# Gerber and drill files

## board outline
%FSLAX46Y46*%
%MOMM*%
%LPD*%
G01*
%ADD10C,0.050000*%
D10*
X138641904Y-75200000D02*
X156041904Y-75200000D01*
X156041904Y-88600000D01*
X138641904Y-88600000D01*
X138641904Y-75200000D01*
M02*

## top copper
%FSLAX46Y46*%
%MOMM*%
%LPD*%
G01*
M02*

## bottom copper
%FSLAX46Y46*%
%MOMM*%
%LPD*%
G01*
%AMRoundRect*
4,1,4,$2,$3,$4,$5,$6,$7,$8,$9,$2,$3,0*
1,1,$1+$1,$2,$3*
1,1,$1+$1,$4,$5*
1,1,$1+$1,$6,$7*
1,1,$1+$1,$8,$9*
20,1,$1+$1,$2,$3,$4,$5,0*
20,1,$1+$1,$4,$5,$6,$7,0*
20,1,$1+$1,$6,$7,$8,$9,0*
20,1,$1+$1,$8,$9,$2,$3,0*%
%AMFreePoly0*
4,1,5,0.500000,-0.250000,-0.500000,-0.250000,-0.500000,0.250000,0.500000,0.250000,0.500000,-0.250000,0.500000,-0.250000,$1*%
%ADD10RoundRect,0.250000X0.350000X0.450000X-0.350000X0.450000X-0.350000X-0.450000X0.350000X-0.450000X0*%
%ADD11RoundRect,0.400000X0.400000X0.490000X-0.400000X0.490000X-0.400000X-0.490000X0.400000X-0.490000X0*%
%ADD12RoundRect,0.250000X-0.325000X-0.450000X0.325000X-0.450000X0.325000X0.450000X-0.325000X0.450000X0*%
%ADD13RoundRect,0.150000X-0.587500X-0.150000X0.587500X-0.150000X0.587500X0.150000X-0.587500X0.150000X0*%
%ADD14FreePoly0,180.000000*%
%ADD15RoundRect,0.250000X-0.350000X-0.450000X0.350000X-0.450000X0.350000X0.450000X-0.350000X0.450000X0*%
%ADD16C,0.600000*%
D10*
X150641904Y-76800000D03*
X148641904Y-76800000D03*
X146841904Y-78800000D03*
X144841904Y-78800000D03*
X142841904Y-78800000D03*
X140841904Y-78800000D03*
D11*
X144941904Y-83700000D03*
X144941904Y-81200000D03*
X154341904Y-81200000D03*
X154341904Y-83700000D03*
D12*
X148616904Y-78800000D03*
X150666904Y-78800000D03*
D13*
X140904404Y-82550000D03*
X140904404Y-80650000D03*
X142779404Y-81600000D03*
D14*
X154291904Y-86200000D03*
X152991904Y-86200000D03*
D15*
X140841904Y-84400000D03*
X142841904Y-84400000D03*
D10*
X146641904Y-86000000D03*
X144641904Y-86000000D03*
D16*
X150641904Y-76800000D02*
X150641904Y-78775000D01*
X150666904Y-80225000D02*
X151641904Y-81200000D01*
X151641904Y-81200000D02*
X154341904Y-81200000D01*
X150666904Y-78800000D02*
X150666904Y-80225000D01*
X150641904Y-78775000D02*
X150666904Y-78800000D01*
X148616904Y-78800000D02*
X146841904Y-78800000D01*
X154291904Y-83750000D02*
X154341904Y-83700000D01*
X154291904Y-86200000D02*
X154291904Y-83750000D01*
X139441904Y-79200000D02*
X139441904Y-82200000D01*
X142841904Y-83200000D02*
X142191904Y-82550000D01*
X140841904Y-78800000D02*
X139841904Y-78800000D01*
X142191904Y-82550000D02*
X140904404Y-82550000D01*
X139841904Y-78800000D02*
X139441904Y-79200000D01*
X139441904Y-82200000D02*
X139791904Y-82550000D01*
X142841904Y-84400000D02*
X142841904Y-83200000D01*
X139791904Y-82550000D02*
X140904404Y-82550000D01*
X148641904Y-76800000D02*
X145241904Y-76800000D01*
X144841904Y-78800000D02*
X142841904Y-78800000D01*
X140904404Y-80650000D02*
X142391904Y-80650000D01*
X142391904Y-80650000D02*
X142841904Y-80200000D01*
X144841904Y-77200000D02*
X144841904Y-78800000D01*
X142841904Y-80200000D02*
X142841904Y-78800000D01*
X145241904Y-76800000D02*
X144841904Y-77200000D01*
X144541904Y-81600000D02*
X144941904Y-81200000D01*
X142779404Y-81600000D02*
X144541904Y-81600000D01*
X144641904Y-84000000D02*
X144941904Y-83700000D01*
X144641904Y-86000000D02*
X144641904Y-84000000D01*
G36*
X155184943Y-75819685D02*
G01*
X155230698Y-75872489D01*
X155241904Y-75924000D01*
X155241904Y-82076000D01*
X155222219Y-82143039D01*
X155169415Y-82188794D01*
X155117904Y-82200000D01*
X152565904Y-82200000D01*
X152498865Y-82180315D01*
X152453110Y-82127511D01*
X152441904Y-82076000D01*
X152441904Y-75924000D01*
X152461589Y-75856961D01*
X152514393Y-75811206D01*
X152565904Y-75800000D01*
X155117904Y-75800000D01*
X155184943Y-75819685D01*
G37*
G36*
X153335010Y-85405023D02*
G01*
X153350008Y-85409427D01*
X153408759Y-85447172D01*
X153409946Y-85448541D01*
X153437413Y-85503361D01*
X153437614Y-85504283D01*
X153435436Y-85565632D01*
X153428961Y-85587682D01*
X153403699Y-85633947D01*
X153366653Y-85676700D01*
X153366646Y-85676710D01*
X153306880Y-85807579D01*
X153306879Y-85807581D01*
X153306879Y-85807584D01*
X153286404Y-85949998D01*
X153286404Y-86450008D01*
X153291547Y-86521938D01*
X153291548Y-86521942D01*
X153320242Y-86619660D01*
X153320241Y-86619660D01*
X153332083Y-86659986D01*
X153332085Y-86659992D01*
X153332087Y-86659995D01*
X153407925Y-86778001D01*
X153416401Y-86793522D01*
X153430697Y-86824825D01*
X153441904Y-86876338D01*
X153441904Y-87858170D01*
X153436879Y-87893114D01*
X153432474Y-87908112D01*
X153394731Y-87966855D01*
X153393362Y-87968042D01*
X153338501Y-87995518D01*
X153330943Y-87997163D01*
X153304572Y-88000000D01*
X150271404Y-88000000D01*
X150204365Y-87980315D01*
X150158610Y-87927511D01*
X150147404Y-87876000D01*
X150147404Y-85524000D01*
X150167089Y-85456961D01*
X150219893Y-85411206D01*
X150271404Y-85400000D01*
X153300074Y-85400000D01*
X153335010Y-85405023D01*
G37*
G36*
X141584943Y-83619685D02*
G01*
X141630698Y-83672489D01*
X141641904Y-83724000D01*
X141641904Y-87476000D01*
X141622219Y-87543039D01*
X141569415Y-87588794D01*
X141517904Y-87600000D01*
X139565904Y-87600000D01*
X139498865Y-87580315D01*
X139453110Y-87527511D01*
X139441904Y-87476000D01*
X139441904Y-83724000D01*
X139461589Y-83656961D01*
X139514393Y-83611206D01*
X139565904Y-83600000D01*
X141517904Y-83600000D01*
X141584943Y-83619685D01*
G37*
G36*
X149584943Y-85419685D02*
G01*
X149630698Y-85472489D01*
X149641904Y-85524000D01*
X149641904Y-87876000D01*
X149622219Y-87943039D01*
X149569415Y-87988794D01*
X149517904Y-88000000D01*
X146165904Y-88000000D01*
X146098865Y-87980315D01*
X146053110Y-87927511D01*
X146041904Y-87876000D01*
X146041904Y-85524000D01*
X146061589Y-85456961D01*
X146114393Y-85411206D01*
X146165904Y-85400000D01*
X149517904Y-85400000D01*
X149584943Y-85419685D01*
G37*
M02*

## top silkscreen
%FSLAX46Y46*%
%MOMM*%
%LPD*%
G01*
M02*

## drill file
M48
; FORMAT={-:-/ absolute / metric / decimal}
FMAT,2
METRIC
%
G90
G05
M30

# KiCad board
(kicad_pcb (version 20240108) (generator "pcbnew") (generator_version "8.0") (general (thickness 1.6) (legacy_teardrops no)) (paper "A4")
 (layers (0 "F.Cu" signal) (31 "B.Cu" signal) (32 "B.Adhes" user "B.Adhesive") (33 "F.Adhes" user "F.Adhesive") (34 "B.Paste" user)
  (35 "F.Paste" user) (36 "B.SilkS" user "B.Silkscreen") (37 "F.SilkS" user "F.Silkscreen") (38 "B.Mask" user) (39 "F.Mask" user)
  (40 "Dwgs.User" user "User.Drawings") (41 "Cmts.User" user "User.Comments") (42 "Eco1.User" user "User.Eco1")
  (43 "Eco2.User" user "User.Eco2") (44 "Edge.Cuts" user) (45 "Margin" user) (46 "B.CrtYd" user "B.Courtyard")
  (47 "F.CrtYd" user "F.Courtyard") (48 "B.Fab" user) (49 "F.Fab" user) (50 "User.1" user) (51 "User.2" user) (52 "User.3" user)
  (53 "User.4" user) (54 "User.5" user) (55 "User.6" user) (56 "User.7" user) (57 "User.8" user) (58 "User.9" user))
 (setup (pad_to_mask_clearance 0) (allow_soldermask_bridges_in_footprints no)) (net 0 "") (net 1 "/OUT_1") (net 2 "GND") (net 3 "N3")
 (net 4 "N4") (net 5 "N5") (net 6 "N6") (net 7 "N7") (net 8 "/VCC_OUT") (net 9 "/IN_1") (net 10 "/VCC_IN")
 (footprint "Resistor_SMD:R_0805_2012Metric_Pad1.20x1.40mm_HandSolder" (layer "B.Cu") (at 149.641904 76.8 180)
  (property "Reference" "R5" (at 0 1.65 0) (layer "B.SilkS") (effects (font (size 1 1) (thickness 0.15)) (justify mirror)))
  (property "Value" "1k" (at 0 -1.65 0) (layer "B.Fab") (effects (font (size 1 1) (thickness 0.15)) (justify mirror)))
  (pad "1" smd roundrect (at -1 0 180) (size 1.2 1.4) (layers "B.Cu" "B.Paste" "B.Mask") (roundrect_rratio 0.208333) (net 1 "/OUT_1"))
  (pad "2" smd roundrect (at 1 0 180) (size 1.2 1.4) (layers "B.Cu" "B.Paste" "B.Mask") (roundrect_rratio 0.208333) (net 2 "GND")))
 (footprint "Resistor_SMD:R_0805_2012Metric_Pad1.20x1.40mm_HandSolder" (layer "B.Cu") (at 145.841904 78.8 180)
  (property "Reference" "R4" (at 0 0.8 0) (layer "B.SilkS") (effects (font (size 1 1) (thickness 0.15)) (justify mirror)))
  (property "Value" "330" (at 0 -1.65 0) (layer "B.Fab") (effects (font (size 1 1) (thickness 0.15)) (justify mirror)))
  (pad "1" smd roundrect (at -1 0 180) (size 1.2 1.4) (layers "B.Cu" "B.Paste" "B.Mask") (roundrect_rratio 0.208333) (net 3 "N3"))
  (pad "2" smd roundrect (at 1 0 180) (size 1.2 1.4) (layers "B.Cu" "B.Paste" "B.Mask") (roundrect_rratio 0.208333) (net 2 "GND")))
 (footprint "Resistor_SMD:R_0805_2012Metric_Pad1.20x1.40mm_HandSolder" (layer "B.Cu") (at 141.841904 78.8 180)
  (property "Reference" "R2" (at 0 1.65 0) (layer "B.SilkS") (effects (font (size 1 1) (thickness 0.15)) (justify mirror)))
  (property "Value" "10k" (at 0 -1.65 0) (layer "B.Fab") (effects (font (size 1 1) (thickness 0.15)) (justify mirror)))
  (pad "1" smd roundrect (at -1 0 180) (size 1.2 1.4) (layers "B.Cu" "B.Paste" "B.Mask") (roundrect_rratio 0.208333) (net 2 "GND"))
  (pad "2" smd roundrect (at 1 0 180) (size 1.2 1.4) (layers "B.Cu" "B.Paste" "B.Mask") (roundrect_rratio 0.208333) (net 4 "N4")))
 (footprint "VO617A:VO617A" (layer "B.Cu") (at 149.641904 82.4 180)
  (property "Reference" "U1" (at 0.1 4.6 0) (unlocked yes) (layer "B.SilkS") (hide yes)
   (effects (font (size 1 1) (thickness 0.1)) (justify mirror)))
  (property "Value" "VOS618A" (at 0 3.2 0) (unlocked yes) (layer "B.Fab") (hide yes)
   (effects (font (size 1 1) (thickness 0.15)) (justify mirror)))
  (pad "1" smd roundrect (at 4.7 -1.3 180) (size 1.6 1.78) (layers "B.Cu" "B.Paste" "B.Mask") (roundrect_rratio 0.25) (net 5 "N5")
   (thermal_bridge_angle 45))
  (pad "2" smd roundrect (at 4.7 1.2 180) (size 1.6 1.78) (layers "B.Cu" "B.Paste" "B.Mask") (roundrect_rratio 0.25) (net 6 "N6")
   (thermal_bridge_angle 45))
  (pad "3" smd roundrect (at -4.7 1.2 180) (size 1.6 1.78) (layers "B.Cu" "B.Paste" "B.Mask") (roundrect_rratio 0.25) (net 1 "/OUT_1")
   (thermal_bridge_angle 45))
  (pad "4" smd roundrect (at -4.7 -1.3 180) (size 1.6 1.78) (layers "B.Cu" "B.Paste" "B.Mask") (roundrect_rratio 0.25) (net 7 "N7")
   (thermal_bridge_angle 45)))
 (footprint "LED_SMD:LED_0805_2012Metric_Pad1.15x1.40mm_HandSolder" (layer "B.Cu") (at 149.641904 78.8)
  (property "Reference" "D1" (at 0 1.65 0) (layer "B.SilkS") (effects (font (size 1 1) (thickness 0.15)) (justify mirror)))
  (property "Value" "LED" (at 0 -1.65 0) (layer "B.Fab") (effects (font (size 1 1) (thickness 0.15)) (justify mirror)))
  (pad "1" smd roundrect (at -1.025 0) (size 1.15 1.4) (layers "B.Cu" "B.Paste" "B.Mask") (roundrect_rratio 0.217391) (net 3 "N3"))
  (pad "2" smd roundrect (at 1.025 0) (size 1.15 1.4) (layers "B.Cu" "B.Paste" "B.Mask") (roundrect_rratio 0.217391) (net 1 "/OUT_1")))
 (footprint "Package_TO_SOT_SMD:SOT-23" (layer "B.Cu") (at 141.841904 81.6)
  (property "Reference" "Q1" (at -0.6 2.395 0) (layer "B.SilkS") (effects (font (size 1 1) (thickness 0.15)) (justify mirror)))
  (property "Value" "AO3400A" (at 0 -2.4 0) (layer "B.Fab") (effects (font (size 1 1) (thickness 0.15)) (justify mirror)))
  (pad "1" smd roundrect (at -0.9375 0.95) (size 1.475 0.6) (layers "B.Cu" "B.Paste" "B.Mask") (roundrect_rratio 0.25) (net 4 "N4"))
  (pad "2" smd roundrect (at -0.9375 -0.95) (size 1.475 0.6) (layers "B.Cu" "B.Paste" "B.Mask") (roundrect_rratio 0.25) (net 2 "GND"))
  (pad "3" smd roundrect (at 0.9375 0) (size 1.475 0.6) (layers "B.Cu" "B.Paste" "B.Mask") (roundrect_rratio 0.25) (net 6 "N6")))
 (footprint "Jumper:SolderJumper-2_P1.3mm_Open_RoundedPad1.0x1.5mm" (layer "B.Cu") (at 153.641904 86.2 180)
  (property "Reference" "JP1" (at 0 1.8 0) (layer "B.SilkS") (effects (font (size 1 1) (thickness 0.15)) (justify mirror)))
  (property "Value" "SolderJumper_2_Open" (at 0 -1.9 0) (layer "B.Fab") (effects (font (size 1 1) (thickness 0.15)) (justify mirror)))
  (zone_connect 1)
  (pad "1" smd custom (at -0.65 0 180) (size 1 0.5) (layers "B.Cu" "B.Mask") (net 7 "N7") (zone_connect 2) (thermal_bridge_angle 45)
   (options (clearance outline) (anchor rect)) (primitives))
  (pad "2" smd custom (at 0.65 0 180) (size 1 0.5) (layers "B.Cu" "B.Mask") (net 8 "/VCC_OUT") (zone_connect 2) (thermal_bridge_angle 45)
   (options (clearance outline) (anchor rect)) (primitives)))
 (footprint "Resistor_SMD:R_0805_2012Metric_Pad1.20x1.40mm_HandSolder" (layer "B.Cu") (at 141.841904 84.4)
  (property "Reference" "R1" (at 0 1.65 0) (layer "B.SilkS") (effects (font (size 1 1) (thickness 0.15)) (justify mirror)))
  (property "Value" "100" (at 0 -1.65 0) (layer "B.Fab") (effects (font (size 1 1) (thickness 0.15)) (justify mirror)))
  (pad "1" smd roundrect (at -1 0) (size 1.2 1.4) (layers "B.Cu" "B.Paste" "B.Mask") (roundrect_rratio 0.208333) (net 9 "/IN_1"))
  (pad "2" smd roundrect (at 1 0) (size 1.2 1.4) (layers "B.Cu" "B.Paste" "B.Mask") (roundrect_rratio 0.208333) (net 4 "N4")))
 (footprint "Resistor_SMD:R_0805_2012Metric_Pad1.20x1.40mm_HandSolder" (layer "B.Cu") (at 145.641904 86 180)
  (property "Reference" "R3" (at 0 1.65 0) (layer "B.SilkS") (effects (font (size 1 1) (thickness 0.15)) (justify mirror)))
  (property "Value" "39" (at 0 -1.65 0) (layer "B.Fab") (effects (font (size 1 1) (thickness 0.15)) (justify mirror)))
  (pad "1" smd roundrect (at -1 0 180) (size 1.2 1.4) (layers "B.Cu" "B.Paste" "B.Mask") (roundrect_rratio 0.208333) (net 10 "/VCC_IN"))
  (pad "2" smd roundrect (at 1 0 180) (size 1.2 1.4) (layers "B.Cu" "B.Paste" "B.Mask") (roundrect_rratio 0.208333) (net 5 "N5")))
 (gr_rect (start 138.641904 75.2) (end 156.041904 88.6) (stroke (width 0.05) (type default)) (fill none) (layer "Edge.Cuts"))
 (segment (start 150.641904 76.8) (end 150.641904 78.775) (width 0.6) (layer "B.Cu") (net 1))
 (segment (start 150.666904 80.225) (end 151.641904 81.2) (width 0.6) (layer "B.Cu") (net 1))
 (segment (start 151.641904 81.2) (end 154.341904 81.2) (width 0.6) (layer "B.Cu") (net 1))
 (segment (start 150.666904 78.8) (end 150.666904 80.225) (width 0.6) (layer "B.Cu") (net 1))
 (segment (start 150.641904 78.775) (end 150.666904 78.8) (width 0.6) (layer "B.Cu") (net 1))
 (segment (start 148.616904 78.8) (end 146.841904 78.8) (width 0.6) (layer "B.Cu") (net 3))
 (segment (start 154.291904 83.75) (end 154.341904 83.7) (width 0.6) (layer "B.Cu") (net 7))
 (segment (start 154.291904 86.2) (end 154.291904 83.75) (width 0.6) (layer "B.Cu") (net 7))
 (segment (start 139.441904 79.2) (end 139.441904 82.2) (width 0.6) (layer "B.Cu") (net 4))
 (segment (start 142.841904 83.2) (end 142.191904 82.55) (width 0.6) (layer "B.Cu") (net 4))
 (segment (start 140.841904 78.8) (end 139.841904 78.8) (width 0.6) (layer "B.Cu") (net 4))
 (segment (start 142.191904 82.55) (end 140.904404 82.55) (width 0.6) (layer "B.Cu") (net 4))
 (segment (start 139.841904 78.8) (end 139.441904 79.2) (width 0.6) (layer "B.Cu") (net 4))
 (segment (start 139.441904 82.2) (end 139.791904 82.55) (width 0.6) (layer "B.Cu") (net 4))
 (segment (start 142.841904 84.4) (end 142.841904 83.2) (width 0.6) (layer "B.Cu") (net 4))
 (segment (start 139.791904 82.55) (end 140.904404 82.55) (width 0.6) (layer "B.Cu") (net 4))
 (segment (start 148.641904 76.8) (end 145.241904 76.8) (width 0.6) (layer "B.Cu") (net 2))
 (segment (start 144.841904 78.8) (end 142.841904 78.8) (width 0.6) (layer "B.Cu") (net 2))
 (segment (start 140.904404 80.65) (end 142.391904 80.65) (width 0.6) (layer "B.Cu") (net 2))
 (segment (start 142.391904 80.65) (end 142.841904 80.2) (width 0.6) (layer "B.Cu") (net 2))
 (segment (start 144.841904 77.2) (end 144.841904 78.8) (width 0.6) (layer "B.Cu") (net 2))
 (segment (start 142.841904 80.2) (end 142.841904 78.8) (width 0.6) (layer "B.Cu") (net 2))
 (segment (start 145.241904 76.8) (end 144.841904 77.2) (width 0.6) (layer "B.Cu") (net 2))
 (segment (start 144.541904 81.6) (end 144.941904 81.2) (width 0.6) (layer "B.Cu") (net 6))
 (segment (start 142.779404 81.6) (end 144.541904 81.6) (width 0.6) (layer "B.Cu") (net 6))
 (segment (start 144.641904 84) (end 144.941904 83.7) (width 0.6) (layer "B.Cu") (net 5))
 (segment (start 144.641904 86) (end 144.641904 84) (width 0.6) (layer "B.Cu") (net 5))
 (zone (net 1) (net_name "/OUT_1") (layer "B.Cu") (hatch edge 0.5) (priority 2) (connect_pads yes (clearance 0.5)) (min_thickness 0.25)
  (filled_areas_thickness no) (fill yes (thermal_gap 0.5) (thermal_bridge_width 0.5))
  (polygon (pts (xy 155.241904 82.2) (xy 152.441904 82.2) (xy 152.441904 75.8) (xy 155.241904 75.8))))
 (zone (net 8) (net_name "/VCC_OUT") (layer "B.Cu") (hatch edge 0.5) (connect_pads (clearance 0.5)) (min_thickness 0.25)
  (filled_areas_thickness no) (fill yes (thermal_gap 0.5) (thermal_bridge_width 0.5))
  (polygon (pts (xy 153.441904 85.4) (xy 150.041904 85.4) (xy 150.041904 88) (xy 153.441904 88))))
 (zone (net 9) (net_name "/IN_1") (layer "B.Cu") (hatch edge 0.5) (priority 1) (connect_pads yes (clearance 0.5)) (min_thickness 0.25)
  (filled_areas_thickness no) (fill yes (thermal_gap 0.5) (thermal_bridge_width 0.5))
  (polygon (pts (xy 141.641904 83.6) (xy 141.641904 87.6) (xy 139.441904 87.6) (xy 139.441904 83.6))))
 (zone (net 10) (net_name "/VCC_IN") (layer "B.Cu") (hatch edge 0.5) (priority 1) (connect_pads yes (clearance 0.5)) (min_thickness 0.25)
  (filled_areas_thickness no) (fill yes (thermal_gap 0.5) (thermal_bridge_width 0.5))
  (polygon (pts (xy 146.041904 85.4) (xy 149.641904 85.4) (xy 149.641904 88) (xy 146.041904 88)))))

